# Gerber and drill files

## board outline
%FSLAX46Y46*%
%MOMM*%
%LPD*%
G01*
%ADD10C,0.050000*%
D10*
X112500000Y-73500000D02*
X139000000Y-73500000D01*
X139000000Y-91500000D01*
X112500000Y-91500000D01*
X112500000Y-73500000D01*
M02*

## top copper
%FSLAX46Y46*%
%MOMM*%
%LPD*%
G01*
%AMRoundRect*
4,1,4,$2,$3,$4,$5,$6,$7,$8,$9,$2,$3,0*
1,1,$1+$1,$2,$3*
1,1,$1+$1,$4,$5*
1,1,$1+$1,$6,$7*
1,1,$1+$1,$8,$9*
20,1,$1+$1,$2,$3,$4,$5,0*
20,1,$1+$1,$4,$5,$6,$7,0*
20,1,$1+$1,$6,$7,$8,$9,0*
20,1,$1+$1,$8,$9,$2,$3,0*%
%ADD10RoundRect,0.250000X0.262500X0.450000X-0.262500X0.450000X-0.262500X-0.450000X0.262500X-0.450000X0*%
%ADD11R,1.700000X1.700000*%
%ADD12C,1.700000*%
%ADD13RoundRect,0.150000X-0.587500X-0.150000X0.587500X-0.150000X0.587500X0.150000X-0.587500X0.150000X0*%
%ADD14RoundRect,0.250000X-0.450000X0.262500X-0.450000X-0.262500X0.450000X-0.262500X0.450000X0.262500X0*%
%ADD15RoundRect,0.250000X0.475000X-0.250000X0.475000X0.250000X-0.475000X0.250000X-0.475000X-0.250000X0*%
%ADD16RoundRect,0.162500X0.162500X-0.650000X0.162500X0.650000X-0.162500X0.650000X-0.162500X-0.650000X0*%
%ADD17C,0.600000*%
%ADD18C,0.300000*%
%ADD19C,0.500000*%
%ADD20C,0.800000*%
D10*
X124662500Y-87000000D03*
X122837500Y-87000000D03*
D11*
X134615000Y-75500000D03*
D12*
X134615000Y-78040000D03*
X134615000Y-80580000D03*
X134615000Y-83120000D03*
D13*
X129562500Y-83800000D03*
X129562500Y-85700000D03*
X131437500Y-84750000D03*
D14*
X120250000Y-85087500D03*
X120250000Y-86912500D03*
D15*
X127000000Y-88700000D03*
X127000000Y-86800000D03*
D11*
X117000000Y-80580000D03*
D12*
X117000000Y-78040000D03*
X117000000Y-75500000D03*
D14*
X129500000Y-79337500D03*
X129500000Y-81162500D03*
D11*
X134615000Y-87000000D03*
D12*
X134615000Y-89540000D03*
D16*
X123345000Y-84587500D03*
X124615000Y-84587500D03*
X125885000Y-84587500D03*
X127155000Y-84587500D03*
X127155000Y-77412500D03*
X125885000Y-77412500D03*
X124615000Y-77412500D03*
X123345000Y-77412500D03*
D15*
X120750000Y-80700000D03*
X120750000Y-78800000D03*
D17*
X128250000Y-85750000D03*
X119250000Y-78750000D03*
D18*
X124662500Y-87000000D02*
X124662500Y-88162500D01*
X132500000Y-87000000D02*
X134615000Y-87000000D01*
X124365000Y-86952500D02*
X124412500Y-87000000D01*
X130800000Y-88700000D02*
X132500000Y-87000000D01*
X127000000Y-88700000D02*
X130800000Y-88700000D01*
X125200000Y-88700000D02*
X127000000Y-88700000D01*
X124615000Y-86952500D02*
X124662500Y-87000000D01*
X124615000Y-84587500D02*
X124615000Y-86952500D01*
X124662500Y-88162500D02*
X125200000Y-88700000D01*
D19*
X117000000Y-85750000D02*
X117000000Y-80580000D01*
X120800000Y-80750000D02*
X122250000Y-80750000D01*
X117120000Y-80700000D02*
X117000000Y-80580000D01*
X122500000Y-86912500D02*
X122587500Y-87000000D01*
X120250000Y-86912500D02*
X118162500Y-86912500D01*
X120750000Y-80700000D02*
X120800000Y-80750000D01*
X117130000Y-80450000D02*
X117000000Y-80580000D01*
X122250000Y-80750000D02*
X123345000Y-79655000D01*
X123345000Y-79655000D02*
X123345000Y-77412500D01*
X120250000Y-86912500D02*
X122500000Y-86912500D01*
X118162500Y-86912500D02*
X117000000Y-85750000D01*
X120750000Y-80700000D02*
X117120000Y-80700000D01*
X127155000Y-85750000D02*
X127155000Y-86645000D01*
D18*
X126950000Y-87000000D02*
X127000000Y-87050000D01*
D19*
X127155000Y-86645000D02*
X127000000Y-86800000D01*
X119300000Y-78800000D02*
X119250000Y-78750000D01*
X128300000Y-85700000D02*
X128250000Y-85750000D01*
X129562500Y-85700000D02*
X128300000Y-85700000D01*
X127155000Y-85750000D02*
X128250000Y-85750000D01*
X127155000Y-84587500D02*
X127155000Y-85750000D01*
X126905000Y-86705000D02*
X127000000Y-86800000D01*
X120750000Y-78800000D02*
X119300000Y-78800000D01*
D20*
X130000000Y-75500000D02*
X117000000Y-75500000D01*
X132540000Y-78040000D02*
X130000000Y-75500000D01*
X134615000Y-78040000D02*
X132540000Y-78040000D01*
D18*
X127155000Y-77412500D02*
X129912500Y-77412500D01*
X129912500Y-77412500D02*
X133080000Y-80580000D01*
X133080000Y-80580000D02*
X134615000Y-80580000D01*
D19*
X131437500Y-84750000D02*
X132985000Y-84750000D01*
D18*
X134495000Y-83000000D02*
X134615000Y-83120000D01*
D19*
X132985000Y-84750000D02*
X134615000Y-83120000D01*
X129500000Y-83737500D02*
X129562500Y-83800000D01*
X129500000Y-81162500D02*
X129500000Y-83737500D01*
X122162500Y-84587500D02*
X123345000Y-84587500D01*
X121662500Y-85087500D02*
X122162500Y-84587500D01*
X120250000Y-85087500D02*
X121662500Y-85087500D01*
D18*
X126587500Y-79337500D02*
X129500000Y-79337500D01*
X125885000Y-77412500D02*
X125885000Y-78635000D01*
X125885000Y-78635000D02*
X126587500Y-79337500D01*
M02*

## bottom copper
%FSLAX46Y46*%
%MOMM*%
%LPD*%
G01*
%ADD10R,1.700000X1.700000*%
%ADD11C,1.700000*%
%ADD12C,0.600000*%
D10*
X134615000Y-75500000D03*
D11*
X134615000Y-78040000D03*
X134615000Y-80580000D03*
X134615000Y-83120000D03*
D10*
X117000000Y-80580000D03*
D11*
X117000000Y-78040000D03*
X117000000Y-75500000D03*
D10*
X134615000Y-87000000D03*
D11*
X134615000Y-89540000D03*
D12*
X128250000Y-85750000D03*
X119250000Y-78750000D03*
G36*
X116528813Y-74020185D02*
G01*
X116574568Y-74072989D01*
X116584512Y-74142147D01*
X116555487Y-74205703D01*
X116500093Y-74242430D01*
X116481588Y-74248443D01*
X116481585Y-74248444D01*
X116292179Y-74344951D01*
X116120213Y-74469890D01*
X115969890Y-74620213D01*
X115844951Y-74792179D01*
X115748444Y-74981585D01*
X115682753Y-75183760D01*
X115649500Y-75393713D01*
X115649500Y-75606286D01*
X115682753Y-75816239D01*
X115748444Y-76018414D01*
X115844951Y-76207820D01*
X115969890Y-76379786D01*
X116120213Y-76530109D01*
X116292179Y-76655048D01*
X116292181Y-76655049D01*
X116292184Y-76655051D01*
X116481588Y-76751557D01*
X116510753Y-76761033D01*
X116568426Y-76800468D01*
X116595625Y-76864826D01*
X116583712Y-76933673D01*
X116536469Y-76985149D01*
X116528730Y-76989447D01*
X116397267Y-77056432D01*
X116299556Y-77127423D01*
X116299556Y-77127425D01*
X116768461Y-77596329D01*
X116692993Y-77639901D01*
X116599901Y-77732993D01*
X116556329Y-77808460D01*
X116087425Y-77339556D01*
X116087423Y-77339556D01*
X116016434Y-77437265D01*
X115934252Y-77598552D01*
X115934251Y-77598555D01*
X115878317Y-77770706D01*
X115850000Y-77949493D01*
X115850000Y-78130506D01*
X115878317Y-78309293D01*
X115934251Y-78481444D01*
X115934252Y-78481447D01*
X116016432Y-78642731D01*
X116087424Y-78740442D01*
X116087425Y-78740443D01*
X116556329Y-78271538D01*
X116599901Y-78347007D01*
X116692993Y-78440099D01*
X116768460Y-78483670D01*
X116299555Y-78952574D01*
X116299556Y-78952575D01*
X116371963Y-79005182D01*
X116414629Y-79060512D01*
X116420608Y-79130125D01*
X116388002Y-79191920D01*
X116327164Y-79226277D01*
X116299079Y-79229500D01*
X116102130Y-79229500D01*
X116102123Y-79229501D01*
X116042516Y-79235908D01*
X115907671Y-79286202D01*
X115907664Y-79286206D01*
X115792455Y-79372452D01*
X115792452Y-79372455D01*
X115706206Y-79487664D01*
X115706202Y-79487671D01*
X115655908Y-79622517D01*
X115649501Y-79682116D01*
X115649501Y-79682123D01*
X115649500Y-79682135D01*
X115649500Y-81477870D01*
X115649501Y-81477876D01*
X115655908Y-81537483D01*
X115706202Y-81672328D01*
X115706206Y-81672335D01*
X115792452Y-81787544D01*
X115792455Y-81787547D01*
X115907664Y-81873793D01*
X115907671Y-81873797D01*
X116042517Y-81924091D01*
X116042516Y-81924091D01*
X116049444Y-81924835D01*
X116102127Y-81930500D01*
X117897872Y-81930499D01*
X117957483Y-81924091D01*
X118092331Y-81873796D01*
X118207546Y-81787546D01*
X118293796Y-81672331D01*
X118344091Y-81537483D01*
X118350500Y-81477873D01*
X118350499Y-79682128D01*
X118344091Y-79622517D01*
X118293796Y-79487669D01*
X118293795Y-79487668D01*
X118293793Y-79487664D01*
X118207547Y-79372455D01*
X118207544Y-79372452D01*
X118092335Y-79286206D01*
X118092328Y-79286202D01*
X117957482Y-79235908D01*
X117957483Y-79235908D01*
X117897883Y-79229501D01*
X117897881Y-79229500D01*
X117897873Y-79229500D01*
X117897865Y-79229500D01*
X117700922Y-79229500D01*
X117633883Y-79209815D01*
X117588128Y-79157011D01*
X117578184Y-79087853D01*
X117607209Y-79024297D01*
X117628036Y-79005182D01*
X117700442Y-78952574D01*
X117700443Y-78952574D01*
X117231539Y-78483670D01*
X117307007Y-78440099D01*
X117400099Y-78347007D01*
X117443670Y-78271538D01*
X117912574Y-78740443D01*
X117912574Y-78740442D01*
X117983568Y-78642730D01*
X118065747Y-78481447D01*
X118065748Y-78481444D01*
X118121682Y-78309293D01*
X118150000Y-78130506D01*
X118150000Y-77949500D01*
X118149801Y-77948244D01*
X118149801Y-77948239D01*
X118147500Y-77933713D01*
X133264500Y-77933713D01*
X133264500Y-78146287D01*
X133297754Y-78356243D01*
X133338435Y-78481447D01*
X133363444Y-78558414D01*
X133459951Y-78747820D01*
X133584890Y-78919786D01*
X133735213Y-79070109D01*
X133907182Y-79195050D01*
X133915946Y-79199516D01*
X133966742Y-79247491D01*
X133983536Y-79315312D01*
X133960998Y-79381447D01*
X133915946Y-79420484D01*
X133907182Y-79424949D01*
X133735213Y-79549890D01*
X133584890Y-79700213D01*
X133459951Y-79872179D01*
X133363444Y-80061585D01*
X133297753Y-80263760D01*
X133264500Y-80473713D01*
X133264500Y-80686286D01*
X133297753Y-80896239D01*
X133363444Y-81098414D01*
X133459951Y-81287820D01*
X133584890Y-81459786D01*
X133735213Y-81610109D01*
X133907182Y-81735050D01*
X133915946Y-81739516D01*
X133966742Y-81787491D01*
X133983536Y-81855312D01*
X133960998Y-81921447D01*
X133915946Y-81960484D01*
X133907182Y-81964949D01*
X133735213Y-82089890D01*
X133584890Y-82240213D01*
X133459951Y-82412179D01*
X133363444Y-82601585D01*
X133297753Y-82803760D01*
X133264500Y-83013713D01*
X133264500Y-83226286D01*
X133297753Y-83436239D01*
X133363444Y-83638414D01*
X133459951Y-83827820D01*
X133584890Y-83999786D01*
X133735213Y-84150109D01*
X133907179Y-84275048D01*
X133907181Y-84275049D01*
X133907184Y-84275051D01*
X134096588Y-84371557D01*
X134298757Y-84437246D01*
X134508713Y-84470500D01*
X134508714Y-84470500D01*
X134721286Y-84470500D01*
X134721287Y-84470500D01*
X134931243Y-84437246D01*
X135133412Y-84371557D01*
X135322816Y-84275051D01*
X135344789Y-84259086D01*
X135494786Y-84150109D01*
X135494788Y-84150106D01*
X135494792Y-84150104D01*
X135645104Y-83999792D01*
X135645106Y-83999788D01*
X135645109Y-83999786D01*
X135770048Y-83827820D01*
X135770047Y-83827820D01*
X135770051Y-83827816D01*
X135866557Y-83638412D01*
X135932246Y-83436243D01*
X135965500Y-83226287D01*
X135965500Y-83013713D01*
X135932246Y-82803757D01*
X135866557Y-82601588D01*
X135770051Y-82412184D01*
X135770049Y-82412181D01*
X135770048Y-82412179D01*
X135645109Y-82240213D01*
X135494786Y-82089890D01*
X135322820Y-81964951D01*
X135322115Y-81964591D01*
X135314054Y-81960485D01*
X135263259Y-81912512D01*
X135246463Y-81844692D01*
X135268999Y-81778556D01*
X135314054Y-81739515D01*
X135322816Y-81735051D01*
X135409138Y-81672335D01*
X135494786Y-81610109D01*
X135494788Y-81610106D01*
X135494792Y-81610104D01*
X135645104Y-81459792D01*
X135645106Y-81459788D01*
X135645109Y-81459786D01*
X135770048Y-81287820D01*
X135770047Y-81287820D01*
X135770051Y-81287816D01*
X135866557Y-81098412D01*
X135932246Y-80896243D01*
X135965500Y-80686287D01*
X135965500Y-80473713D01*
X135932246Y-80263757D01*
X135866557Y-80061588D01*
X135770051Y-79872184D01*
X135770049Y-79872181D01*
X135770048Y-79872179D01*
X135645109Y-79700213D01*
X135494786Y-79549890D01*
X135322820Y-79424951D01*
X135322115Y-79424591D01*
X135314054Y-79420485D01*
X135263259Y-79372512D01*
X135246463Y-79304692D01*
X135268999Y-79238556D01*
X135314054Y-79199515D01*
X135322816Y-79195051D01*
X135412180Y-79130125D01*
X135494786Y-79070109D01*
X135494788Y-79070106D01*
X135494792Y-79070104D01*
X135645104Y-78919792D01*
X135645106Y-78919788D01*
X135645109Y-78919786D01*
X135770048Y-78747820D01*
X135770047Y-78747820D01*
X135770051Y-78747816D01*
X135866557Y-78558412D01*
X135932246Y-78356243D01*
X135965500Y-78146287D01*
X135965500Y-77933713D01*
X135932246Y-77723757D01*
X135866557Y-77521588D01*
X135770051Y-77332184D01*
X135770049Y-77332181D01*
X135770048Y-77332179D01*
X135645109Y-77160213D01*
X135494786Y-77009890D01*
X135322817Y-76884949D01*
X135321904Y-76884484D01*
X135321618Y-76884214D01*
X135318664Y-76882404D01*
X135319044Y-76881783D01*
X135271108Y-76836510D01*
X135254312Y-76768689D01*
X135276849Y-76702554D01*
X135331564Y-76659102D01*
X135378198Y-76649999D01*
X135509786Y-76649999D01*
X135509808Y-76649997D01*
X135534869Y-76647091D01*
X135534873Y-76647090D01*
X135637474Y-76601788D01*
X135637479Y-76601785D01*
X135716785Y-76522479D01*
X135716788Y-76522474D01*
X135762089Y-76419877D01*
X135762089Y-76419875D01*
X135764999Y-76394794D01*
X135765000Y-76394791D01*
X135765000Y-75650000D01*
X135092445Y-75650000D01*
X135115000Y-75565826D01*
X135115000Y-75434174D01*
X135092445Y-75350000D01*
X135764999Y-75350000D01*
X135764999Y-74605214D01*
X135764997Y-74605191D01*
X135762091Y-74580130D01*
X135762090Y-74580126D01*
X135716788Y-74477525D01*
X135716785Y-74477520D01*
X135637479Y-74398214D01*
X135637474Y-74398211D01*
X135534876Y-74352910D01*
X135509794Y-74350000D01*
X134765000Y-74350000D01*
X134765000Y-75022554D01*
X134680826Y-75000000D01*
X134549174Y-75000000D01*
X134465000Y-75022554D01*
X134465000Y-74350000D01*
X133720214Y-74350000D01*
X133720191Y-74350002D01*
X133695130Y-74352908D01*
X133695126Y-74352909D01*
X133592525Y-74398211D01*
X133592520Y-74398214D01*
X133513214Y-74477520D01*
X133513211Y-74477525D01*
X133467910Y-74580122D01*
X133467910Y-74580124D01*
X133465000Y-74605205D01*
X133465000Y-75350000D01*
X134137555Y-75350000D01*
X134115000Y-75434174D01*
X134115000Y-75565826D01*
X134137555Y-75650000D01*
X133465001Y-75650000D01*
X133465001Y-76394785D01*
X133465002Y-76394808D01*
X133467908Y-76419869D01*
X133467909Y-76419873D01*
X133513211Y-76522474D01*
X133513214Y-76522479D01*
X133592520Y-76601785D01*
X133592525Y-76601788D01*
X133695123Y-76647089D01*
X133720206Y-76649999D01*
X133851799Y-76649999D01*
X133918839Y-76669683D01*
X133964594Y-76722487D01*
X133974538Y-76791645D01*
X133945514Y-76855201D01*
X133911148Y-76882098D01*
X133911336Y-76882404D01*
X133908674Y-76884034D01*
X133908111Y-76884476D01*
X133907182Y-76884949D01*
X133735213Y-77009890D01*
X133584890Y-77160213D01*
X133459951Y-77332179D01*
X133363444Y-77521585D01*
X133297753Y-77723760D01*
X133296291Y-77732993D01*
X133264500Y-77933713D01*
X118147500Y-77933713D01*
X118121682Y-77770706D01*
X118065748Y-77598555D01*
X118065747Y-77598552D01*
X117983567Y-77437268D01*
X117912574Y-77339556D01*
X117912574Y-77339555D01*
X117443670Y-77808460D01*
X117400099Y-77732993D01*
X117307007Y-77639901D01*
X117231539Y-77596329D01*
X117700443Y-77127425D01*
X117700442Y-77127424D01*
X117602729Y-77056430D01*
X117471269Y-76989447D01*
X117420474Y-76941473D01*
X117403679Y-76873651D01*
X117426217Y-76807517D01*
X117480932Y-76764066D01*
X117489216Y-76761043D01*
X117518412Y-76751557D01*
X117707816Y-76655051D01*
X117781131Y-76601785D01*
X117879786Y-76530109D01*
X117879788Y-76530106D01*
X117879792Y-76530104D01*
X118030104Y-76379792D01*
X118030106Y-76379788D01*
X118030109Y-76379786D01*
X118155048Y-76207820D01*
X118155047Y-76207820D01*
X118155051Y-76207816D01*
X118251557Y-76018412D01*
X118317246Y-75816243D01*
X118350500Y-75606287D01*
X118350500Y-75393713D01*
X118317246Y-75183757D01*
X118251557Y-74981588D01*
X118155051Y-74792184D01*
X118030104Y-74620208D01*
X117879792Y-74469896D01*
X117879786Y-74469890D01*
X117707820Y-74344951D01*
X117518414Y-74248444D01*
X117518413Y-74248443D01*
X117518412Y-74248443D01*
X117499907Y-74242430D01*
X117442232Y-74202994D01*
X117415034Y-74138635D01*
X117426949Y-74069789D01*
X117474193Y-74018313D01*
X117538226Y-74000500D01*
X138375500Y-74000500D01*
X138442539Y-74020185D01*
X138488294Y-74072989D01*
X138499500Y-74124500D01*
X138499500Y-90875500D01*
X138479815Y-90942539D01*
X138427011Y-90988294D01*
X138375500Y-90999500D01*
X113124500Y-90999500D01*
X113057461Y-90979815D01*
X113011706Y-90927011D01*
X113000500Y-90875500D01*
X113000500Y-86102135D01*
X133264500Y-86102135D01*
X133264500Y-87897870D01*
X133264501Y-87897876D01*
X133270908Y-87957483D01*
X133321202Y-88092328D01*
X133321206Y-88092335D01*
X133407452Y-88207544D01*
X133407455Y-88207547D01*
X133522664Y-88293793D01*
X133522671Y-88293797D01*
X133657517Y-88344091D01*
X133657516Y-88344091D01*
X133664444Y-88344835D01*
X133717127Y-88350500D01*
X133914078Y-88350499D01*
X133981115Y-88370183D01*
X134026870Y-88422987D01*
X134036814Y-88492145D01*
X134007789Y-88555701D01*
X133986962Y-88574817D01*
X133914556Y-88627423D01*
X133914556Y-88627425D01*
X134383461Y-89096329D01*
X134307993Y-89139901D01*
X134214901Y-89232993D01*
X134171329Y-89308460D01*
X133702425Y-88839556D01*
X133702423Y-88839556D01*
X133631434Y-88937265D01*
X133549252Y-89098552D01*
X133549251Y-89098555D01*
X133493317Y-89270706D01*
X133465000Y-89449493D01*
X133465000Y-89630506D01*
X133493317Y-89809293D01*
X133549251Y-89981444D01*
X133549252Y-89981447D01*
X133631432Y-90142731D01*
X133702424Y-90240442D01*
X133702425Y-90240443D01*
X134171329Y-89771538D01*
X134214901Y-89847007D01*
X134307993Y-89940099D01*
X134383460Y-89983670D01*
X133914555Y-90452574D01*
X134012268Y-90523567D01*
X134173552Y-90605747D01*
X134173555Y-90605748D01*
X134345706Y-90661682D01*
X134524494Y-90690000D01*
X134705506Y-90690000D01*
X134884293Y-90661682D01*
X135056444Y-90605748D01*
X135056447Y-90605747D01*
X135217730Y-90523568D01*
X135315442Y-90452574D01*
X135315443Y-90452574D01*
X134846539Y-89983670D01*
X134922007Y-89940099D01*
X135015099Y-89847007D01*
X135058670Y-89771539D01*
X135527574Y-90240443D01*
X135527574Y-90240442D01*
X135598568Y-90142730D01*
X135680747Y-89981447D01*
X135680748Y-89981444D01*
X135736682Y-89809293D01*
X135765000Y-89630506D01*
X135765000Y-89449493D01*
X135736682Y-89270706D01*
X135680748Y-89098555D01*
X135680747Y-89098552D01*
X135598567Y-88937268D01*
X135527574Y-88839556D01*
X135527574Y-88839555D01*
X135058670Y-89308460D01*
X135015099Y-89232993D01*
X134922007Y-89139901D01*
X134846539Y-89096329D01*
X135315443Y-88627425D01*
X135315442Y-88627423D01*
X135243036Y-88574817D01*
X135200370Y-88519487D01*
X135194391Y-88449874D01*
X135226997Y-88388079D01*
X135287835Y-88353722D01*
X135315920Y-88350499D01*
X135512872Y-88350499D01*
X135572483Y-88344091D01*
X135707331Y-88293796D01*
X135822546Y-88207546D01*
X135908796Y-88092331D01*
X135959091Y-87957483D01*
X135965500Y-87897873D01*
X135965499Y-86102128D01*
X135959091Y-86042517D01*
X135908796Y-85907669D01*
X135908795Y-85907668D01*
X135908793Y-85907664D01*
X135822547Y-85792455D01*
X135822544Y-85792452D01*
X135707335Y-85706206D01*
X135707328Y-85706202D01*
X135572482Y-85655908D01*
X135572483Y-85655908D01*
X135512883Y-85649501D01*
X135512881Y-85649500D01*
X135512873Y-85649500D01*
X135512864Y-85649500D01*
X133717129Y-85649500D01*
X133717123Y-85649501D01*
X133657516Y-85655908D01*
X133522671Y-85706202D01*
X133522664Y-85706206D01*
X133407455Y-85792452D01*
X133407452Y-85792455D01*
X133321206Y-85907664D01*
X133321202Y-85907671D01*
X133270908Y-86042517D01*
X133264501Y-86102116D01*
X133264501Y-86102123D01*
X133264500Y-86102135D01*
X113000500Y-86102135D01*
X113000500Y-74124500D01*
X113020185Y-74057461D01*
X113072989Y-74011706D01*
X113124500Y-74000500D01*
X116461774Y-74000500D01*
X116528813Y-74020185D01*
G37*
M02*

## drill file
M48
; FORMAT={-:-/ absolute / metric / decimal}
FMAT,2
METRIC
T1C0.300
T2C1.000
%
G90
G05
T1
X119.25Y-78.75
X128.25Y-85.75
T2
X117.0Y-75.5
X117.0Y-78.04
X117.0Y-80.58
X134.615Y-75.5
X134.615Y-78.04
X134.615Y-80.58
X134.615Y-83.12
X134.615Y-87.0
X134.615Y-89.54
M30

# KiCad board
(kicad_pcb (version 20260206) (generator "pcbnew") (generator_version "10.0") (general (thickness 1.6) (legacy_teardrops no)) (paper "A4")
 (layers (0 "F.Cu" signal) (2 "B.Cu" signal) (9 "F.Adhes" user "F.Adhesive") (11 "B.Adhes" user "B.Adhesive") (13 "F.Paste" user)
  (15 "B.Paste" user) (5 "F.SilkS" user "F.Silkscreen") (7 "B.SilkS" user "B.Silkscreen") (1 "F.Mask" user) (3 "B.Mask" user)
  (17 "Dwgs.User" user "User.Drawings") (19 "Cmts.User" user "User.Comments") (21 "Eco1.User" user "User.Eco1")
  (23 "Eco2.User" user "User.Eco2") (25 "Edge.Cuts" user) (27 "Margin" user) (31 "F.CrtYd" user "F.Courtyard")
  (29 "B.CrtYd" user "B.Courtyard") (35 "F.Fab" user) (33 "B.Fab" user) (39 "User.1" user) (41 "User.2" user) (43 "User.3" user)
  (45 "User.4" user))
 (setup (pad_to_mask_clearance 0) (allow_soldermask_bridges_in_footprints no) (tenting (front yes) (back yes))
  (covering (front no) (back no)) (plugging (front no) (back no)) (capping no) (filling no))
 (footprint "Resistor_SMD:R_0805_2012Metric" (layer "F.Cu") (at 123.75 87 180)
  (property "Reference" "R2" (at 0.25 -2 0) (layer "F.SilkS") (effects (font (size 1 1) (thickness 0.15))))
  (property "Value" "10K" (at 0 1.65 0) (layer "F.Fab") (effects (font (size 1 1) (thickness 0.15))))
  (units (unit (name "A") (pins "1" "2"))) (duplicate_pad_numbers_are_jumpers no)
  (pad "1" smd roundrect (at -0.9125 0 180) (size 1.025 1.4) (layers "F.Cu" "F.Mask" "F.Paste") (roundrect_rratio 0.243902)
   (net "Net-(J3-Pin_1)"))
  (pad "2" smd roundrect (at 0.9125 0 180) (size 1.025 1.4) (layers "F.Cu" "F.Mask" "F.Paste") (roundrect_rratio 0.243902) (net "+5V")))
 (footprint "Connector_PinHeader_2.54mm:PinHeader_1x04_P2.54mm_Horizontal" (layer "F.Cu") (at 134.615 75.5)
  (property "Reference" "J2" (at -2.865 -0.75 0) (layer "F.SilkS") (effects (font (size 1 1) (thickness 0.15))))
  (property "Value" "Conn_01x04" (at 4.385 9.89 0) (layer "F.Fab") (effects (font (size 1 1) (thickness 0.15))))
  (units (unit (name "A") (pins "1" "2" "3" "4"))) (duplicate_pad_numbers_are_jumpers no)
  (pad "1" thru_hole rect (at 0 0) (size 1.7 1.7) (drill 1) (layers "*.Cu" "*.Mask") (remove_unused_layers no) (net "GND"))
  (pad "2" thru_hole circle (at 0 2.54) (size 1.7 1.7) (drill 1) (layers "*.Cu" "*.Mask") (remove_unused_layers no) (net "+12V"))
  (pad "3" thru_hole circle (at 0 5.08) (size 1.7 1.7) (drill 1) (layers "*.Cu" "*.Mask") (remove_unused_layers no) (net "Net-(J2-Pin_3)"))
  (pad "4" thru_hole circle (at 0 7.62) (size 1.7 1.7) (drill 1) (layers "*.Cu" "*.Mask") (remove_unused_layers no) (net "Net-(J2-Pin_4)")))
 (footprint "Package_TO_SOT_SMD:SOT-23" (layer "F.Cu") (at 130.5 84.75)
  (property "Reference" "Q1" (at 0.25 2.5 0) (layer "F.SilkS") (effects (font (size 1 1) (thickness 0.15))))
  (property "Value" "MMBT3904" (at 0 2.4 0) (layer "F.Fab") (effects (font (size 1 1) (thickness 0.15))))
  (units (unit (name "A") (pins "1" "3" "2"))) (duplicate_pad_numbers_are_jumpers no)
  (pad "1" smd roundrect (at -0.9375 -0.95) (size 1.475 0.6) (layers "F.Cu" "F.Mask" "F.Paste") (roundrect_rratio 0.25) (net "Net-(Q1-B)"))
  (pad "2" smd roundrect (at -0.9375 0.95) (size 1.475 0.6) (layers "F.Cu" "F.Mask" "F.Paste") (roundrect_rratio 0.25) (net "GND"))
  (pad "3" smd roundrect (at 0.9375 0) (size 1.475 0.6) (layers "F.Cu" "F.Mask" "F.Paste") (roundrect_rratio 0.25) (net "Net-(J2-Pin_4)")))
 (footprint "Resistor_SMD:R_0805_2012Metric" (layer "F.Cu") (at 120.25 86 -90)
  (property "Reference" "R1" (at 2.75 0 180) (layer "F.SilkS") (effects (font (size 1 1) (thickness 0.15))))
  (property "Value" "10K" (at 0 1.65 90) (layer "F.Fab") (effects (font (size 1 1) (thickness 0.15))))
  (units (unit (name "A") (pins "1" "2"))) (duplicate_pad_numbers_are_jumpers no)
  (pad "1" smd roundrect (at -0.9125 0 270) (size 1.025 1.4) (layers "F.Cu" "F.Mask" "F.Paste") (roundrect_rratio 0.243902)
   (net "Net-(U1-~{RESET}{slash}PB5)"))
  (pad "2" smd roundrect (at 0.9125 0 270) (size 1.025 1.4) (layers "F.Cu" "F.Mask" "F.Paste") (roundrect_rratio 0.243902) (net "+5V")))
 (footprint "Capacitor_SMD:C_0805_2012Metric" (layer "F.Cu") (at 127 87.75 90)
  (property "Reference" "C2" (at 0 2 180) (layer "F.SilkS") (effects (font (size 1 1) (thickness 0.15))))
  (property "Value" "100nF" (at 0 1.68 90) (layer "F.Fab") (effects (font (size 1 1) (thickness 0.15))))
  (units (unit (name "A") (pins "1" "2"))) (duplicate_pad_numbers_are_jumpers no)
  (pad "1" smd roundrect (at -0.95 0 90) (size 1 1.45) (layers "F.Cu" "F.Mask" "F.Paste") (roundrect_rratio 0.25) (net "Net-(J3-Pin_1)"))
  (pad "2" smd roundrect (at 0.95 0 90) (size 1 1.45) (layers "F.Cu" "F.Mask" "F.Paste") (roundrect_rratio 0.25) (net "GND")))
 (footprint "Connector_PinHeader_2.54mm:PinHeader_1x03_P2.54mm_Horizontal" (layer "F.Cu") (at 117 80.58 180)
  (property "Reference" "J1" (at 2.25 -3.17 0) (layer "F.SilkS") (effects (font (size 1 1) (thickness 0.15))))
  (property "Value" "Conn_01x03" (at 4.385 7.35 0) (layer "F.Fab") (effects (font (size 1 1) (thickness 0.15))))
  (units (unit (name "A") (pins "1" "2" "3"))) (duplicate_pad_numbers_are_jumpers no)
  (pad "1" thru_hole rect (at 0 0 180) (size 1.7 1.7) (drill 1) (layers "*.Cu" "*.Mask") (remove_unused_layers no) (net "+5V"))
  (pad "2" thru_hole circle (at 0 2.54 180) (size 1.7 1.7) (drill 1) (layers "*.Cu" "*.Mask") (remove_unused_layers no) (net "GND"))
  (pad "3" thru_hole circle (at 0 5.08 180) (size 1.7 1.7) (drill 1) (layers "*.Cu" "*.Mask") (remove_unused_layers no) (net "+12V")))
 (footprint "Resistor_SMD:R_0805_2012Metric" (layer "F.Cu") (at 129.5 80.25 -90)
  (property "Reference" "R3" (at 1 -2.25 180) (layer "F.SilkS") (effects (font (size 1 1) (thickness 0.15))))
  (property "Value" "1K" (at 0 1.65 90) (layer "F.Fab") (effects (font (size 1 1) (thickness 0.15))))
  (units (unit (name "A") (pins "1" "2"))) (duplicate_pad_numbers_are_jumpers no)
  (pad "1" smd roundrect (at -0.9125 0 270) (size 1.025 1.4) (layers "F.Cu" "F.Mask" "F.Paste") (roundrect_rratio 0.243902)
   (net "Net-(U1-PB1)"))
  (pad "2" smd roundrect (at 0.9125 0 270) (size 1.025 1.4) (layers "F.Cu" "F.Mask" "F.Paste") (roundrect_rratio 0.243902)
   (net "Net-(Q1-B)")))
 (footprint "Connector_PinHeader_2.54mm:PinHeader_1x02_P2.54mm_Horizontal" (layer "F.Cu") (at 134.615 87)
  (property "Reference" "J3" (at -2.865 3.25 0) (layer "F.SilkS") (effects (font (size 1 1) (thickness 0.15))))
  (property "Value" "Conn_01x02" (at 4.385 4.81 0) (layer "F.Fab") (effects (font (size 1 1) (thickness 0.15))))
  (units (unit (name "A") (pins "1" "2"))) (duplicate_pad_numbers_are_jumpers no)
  (pad "1" thru_hole rect (at 0 0) (size 1.7 1.7) (drill 1) (layers "*.Cu" "*.Mask") (remove_unused_layers no) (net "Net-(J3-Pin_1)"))
  (pad "2" thru_hole circle (at 0 2.54) (size 1.7 1.7) (drill 1) (layers "*.Cu" "*.Mask") (remove_unused_layers no) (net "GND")))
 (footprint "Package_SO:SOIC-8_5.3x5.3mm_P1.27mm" (layer "F.Cu") (at 125.25 81 90)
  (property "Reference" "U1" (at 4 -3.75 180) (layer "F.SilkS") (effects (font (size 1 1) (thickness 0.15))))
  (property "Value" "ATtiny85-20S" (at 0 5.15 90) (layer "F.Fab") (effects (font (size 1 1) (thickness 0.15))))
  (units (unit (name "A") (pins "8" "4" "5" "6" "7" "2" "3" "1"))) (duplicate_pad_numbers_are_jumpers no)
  (pad "1" smd roundrect (at -3.5875 -1.905 90) (size 1.625 0.65) (layers "F.Cu" "F.Mask" "F.Paste") (roundrect_rratio 0.25)
   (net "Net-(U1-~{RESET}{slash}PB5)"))
  (pad "2" smd roundrect (at -3.5875 -0.635 90) (size 1.625 0.65) (layers "F.Cu" "F.Mask" "F.Paste") (roundrect_rratio 0.25)
   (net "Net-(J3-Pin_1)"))
  (pad "3" smd roundrect (at -3.5875 0.635 90) (size 1.625 0.65) (layers "F.Cu" "F.Mask" "F.Paste") (roundrect_rratio 0.25)
   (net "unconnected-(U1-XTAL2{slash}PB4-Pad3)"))
  (pad "4" smd roundrect (at -3.5875 1.905 90) (size 1.625 0.65) (layers "F.Cu" "F.Mask" "F.Paste") (roundrect_rratio 0.25) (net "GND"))
  (pad "5" smd roundrect (at 3.5875 1.905 90) (size 1.625 0.65) (layers "F.Cu" "F.Mask" "F.Paste") (roundrect_rratio 0.25)
   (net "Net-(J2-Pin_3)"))
  (pad "6" smd roundrect (at 3.5875 0.635 90) (size 1.625 0.65) (layers "F.Cu" "F.Mask" "F.Paste") (roundrect_rratio 0.25)
   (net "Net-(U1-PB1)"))
  (pad "7" smd roundrect (at 3.5875 -0.635 90) (size 1.625 0.65) (layers "F.Cu" "F.Mask" "F.Paste") (roundrect_rratio 0.25)
   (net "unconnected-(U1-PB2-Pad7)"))
  (pad "8" smd roundrect (at 3.5875 -1.905 90) (size 1.625 0.65) (layers "F.Cu" "F.Mask" "F.Paste") (roundrect_rratio 0.25) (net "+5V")))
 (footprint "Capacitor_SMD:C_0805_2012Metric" (layer "F.Cu") (at 120.75 79.75 90)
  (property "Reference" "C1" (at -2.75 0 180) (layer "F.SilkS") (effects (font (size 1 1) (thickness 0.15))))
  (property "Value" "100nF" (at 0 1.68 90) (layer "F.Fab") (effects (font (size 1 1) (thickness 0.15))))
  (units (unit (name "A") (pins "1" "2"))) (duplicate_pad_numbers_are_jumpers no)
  (pad "1" smd roundrect (at -0.95 0 90) (size 1 1.45) (layers "F.Cu" "F.Mask" "F.Paste") (roundrect_rratio 0.25) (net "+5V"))
  (pad "2" smd roundrect (at 0.95 0 90) (size 1 1.45) (layers "F.Cu" "F.Mask" "F.Paste") (roundrect_rratio 0.25) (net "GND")))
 (gr_rect (start 112.5 73.5) (end 139 91.5) (stroke (width 0.05) (type default)) (fill no) (layer "Edge.Cuts"))
 (segment (start 124.6625 87) (end 124.6625 88.1625) (width 0.3) (layer "F.Cu") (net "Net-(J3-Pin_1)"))
 (segment (start 132.5 87) (end 134.615 87) (width 0.3) (layer "F.Cu") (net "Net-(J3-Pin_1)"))
 (segment (start 124.365 86.9525) (end 124.4125 87) (width 0.3) (layer "F.Cu") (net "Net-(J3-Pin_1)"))
 (segment (start 130.8 88.7) (end 132.5 87) (width 0.3) (layer "F.Cu") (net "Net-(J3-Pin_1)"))
 (segment (start 127 88.7) (end 130.8 88.7) (width 0.3) (layer "F.Cu") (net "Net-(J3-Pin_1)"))
 (segment (start 125.2 88.7) (end 127 88.7) (width 0.3) (layer "F.Cu") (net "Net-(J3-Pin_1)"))
 (segment (start 124.615 86.9525) (end 124.6625 87) (width 0.3) (layer "F.Cu") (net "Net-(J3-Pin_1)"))
 (segment (start 124.615 84.5875) (end 124.615 86.9525) (width 0.3) (layer "F.Cu") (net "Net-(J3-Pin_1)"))
 (segment (start 124.6625 88.1625) (end 125.2 88.7) (width 0.3) (layer "F.Cu") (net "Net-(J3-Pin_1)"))
 (segment (start 117 85.75) (end 117 80.58) (width 0.5) (layer "F.Cu") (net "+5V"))
 (segment (start 120.8 80.75) (end 122.25 80.75) (width 0.5) (layer "F.Cu") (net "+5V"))
 (segment (start 117.12 80.7) (end 117 80.58) (width 0.5) (layer "F.Cu") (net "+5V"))
 (segment (start 122.5 86.9125) (end 122.5875 87) (width 0.5) (layer "F.Cu") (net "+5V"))
 (segment (start 120.25 86.9125) (end 118.1625 86.9125) (width 0.5) (layer "F.Cu") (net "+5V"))
 (segment (start 120.75 80.7) (end 120.8 80.75) (width 0.5) (layer "F.Cu") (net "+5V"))
 (segment (start 117.13 80.45) (end 117 80.58) (width 0.5) (layer "F.Cu") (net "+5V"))
 (segment (start 122.25 80.75) (end 123.345 79.655) (width 0.5) (layer "F.Cu") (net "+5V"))
 (segment (start 123.345 79.655) (end 123.345 77.4125) (width 0.5) (layer "F.Cu") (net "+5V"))
 (segment (start 120.25 86.9125) (end 122.5 86.9125) (width 0.5) (layer "F.Cu") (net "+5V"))
 (segment (start 118.1625 86.9125) (end 117 85.75) (width 0.5) (layer "F.Cu") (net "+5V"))
 (segment (start 120.75 80.7) (end 117.12 80.7) (width 0.5) (layer "F.Cu") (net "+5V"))
 (segment (start 127.155 85.75) (end 127.155 86.645) (width 0.5) (layer "F.Cu") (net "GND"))
 (segment (start 126.95 87) (end 127 87.05) (width 0.3) (layer "F.Cu") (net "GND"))
 (segment (start 127.155 86.645) (end 127 86.8) (width 0.5) (layer "F.Cu") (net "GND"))
 (segment (start 119.3 78.8) (end 119.25 78.75) (width 0.5) (layer "F.Cu") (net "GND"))
 (segment (start 128.3 85.7) (end 128.25 85.75) (width 0.5) (layer "F.Cu") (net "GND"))
 (segment (start 129.5625 85.7) (end 128.3 85.7) (width 0.5) (layer "F.Cu") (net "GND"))
 (segment (start 127.155 85.75) (end 128.25 85.75) (width 0.5) (layer "F.Cu") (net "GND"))
 (segment (start 127.155 84.5875) (end 127.155 85.75) (width 0.5) (layer "F.Cu") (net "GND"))
 (segment (start 126.905 86.705) (end 127 86.8) (width 0.5) (layer "F.Cu") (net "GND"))
 (segment (start 120.75 78.8) (end 119.3 78.8) (width 0.5) (layer "F.Cu") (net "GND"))
 (via (at 128.25 85.75) (size 0.6) (drill 0.3) (layers "F.Cu" "B.Cu") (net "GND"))
 (via (at 119.25 78.75) (size 0.6) (drill 0.3) (layers "F.Cu" "B.Cu") (free yes) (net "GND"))
 (segment (start 130 75.5) (end 117 75.5) (width 0.8) (layer "F.Cu") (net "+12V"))
 (segment (start 132.54 78.04) (end 130 75.5) (width 0.8) (layer "F.Cu") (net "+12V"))
 (segment (start 134.615 78.04) (end 132.54 78.04) (width 0.8) (layer "F.Cu") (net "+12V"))
 (segment (start 127.155 77.4125) (end 129.9125 77.4125) (width 0.3) (layer "F.Cu") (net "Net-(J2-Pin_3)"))
 (segment (start 129.9125 77.4125) (end 133.08 80.58) (width 0.3) (layer "F.Cu") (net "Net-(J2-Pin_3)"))
 (segment (start 133.08 80.58) (end 134.615 80.58) (width 0.3) (layer "F.Cu") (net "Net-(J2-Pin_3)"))
 (segment (start 131.4375 84.75) (end 132.985 84.75) (width 0.5) (layer "F.Cu") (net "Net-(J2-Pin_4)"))
 (segment (start 134.495 83) (end 134.615 83.12) (width 0.3) (layer "F.Cu") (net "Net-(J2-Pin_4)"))
 (segment (start 132.985 84.75) (end 134.615 83.12) (width 0.5) (layer "F.Cu") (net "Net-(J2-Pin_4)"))
 (segment (start 129.5 83.7375) (end 129.5625 83.8) (width 0.5) (layer "F.Cu") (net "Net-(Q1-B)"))
 (segment (start 129.5 81.1625) (end 129.5 83.7375) (width 0.5) (layer "F.Cu") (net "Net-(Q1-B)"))
 (segment (start 122.1625 84.5875) (end 123.345 84.5875) (width 0.5) (layer "F.Cu") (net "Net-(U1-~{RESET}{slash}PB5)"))
 (segment (start 121.6625 85.0875) (end 122.1625 84.5875) (width 0.5) (layer "F.Cu") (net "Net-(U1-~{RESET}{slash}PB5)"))
 (segment (start 120.25 85.0875) (end 121.6625 85.0875) (width 0.5) (layer "F.Cu") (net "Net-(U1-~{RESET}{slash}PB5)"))
 (segment (start 126.5875 79.3375) (end 129.5 79.3375) (width 0.3) (layer "F.Cu") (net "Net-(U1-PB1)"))
 (segment (start 125.885 77.4125) (end 125.885 78.635) (width 0.3) (layer "F.Cu") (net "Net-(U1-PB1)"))
 (segment (start 125.885 78.635) (end 126.5875 79.3375) (width 0.3) (layer "F.Cu") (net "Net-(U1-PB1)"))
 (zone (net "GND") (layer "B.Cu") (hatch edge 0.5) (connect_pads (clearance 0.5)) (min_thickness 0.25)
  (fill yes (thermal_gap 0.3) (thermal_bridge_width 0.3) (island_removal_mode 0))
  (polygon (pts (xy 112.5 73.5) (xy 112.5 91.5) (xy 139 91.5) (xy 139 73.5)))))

